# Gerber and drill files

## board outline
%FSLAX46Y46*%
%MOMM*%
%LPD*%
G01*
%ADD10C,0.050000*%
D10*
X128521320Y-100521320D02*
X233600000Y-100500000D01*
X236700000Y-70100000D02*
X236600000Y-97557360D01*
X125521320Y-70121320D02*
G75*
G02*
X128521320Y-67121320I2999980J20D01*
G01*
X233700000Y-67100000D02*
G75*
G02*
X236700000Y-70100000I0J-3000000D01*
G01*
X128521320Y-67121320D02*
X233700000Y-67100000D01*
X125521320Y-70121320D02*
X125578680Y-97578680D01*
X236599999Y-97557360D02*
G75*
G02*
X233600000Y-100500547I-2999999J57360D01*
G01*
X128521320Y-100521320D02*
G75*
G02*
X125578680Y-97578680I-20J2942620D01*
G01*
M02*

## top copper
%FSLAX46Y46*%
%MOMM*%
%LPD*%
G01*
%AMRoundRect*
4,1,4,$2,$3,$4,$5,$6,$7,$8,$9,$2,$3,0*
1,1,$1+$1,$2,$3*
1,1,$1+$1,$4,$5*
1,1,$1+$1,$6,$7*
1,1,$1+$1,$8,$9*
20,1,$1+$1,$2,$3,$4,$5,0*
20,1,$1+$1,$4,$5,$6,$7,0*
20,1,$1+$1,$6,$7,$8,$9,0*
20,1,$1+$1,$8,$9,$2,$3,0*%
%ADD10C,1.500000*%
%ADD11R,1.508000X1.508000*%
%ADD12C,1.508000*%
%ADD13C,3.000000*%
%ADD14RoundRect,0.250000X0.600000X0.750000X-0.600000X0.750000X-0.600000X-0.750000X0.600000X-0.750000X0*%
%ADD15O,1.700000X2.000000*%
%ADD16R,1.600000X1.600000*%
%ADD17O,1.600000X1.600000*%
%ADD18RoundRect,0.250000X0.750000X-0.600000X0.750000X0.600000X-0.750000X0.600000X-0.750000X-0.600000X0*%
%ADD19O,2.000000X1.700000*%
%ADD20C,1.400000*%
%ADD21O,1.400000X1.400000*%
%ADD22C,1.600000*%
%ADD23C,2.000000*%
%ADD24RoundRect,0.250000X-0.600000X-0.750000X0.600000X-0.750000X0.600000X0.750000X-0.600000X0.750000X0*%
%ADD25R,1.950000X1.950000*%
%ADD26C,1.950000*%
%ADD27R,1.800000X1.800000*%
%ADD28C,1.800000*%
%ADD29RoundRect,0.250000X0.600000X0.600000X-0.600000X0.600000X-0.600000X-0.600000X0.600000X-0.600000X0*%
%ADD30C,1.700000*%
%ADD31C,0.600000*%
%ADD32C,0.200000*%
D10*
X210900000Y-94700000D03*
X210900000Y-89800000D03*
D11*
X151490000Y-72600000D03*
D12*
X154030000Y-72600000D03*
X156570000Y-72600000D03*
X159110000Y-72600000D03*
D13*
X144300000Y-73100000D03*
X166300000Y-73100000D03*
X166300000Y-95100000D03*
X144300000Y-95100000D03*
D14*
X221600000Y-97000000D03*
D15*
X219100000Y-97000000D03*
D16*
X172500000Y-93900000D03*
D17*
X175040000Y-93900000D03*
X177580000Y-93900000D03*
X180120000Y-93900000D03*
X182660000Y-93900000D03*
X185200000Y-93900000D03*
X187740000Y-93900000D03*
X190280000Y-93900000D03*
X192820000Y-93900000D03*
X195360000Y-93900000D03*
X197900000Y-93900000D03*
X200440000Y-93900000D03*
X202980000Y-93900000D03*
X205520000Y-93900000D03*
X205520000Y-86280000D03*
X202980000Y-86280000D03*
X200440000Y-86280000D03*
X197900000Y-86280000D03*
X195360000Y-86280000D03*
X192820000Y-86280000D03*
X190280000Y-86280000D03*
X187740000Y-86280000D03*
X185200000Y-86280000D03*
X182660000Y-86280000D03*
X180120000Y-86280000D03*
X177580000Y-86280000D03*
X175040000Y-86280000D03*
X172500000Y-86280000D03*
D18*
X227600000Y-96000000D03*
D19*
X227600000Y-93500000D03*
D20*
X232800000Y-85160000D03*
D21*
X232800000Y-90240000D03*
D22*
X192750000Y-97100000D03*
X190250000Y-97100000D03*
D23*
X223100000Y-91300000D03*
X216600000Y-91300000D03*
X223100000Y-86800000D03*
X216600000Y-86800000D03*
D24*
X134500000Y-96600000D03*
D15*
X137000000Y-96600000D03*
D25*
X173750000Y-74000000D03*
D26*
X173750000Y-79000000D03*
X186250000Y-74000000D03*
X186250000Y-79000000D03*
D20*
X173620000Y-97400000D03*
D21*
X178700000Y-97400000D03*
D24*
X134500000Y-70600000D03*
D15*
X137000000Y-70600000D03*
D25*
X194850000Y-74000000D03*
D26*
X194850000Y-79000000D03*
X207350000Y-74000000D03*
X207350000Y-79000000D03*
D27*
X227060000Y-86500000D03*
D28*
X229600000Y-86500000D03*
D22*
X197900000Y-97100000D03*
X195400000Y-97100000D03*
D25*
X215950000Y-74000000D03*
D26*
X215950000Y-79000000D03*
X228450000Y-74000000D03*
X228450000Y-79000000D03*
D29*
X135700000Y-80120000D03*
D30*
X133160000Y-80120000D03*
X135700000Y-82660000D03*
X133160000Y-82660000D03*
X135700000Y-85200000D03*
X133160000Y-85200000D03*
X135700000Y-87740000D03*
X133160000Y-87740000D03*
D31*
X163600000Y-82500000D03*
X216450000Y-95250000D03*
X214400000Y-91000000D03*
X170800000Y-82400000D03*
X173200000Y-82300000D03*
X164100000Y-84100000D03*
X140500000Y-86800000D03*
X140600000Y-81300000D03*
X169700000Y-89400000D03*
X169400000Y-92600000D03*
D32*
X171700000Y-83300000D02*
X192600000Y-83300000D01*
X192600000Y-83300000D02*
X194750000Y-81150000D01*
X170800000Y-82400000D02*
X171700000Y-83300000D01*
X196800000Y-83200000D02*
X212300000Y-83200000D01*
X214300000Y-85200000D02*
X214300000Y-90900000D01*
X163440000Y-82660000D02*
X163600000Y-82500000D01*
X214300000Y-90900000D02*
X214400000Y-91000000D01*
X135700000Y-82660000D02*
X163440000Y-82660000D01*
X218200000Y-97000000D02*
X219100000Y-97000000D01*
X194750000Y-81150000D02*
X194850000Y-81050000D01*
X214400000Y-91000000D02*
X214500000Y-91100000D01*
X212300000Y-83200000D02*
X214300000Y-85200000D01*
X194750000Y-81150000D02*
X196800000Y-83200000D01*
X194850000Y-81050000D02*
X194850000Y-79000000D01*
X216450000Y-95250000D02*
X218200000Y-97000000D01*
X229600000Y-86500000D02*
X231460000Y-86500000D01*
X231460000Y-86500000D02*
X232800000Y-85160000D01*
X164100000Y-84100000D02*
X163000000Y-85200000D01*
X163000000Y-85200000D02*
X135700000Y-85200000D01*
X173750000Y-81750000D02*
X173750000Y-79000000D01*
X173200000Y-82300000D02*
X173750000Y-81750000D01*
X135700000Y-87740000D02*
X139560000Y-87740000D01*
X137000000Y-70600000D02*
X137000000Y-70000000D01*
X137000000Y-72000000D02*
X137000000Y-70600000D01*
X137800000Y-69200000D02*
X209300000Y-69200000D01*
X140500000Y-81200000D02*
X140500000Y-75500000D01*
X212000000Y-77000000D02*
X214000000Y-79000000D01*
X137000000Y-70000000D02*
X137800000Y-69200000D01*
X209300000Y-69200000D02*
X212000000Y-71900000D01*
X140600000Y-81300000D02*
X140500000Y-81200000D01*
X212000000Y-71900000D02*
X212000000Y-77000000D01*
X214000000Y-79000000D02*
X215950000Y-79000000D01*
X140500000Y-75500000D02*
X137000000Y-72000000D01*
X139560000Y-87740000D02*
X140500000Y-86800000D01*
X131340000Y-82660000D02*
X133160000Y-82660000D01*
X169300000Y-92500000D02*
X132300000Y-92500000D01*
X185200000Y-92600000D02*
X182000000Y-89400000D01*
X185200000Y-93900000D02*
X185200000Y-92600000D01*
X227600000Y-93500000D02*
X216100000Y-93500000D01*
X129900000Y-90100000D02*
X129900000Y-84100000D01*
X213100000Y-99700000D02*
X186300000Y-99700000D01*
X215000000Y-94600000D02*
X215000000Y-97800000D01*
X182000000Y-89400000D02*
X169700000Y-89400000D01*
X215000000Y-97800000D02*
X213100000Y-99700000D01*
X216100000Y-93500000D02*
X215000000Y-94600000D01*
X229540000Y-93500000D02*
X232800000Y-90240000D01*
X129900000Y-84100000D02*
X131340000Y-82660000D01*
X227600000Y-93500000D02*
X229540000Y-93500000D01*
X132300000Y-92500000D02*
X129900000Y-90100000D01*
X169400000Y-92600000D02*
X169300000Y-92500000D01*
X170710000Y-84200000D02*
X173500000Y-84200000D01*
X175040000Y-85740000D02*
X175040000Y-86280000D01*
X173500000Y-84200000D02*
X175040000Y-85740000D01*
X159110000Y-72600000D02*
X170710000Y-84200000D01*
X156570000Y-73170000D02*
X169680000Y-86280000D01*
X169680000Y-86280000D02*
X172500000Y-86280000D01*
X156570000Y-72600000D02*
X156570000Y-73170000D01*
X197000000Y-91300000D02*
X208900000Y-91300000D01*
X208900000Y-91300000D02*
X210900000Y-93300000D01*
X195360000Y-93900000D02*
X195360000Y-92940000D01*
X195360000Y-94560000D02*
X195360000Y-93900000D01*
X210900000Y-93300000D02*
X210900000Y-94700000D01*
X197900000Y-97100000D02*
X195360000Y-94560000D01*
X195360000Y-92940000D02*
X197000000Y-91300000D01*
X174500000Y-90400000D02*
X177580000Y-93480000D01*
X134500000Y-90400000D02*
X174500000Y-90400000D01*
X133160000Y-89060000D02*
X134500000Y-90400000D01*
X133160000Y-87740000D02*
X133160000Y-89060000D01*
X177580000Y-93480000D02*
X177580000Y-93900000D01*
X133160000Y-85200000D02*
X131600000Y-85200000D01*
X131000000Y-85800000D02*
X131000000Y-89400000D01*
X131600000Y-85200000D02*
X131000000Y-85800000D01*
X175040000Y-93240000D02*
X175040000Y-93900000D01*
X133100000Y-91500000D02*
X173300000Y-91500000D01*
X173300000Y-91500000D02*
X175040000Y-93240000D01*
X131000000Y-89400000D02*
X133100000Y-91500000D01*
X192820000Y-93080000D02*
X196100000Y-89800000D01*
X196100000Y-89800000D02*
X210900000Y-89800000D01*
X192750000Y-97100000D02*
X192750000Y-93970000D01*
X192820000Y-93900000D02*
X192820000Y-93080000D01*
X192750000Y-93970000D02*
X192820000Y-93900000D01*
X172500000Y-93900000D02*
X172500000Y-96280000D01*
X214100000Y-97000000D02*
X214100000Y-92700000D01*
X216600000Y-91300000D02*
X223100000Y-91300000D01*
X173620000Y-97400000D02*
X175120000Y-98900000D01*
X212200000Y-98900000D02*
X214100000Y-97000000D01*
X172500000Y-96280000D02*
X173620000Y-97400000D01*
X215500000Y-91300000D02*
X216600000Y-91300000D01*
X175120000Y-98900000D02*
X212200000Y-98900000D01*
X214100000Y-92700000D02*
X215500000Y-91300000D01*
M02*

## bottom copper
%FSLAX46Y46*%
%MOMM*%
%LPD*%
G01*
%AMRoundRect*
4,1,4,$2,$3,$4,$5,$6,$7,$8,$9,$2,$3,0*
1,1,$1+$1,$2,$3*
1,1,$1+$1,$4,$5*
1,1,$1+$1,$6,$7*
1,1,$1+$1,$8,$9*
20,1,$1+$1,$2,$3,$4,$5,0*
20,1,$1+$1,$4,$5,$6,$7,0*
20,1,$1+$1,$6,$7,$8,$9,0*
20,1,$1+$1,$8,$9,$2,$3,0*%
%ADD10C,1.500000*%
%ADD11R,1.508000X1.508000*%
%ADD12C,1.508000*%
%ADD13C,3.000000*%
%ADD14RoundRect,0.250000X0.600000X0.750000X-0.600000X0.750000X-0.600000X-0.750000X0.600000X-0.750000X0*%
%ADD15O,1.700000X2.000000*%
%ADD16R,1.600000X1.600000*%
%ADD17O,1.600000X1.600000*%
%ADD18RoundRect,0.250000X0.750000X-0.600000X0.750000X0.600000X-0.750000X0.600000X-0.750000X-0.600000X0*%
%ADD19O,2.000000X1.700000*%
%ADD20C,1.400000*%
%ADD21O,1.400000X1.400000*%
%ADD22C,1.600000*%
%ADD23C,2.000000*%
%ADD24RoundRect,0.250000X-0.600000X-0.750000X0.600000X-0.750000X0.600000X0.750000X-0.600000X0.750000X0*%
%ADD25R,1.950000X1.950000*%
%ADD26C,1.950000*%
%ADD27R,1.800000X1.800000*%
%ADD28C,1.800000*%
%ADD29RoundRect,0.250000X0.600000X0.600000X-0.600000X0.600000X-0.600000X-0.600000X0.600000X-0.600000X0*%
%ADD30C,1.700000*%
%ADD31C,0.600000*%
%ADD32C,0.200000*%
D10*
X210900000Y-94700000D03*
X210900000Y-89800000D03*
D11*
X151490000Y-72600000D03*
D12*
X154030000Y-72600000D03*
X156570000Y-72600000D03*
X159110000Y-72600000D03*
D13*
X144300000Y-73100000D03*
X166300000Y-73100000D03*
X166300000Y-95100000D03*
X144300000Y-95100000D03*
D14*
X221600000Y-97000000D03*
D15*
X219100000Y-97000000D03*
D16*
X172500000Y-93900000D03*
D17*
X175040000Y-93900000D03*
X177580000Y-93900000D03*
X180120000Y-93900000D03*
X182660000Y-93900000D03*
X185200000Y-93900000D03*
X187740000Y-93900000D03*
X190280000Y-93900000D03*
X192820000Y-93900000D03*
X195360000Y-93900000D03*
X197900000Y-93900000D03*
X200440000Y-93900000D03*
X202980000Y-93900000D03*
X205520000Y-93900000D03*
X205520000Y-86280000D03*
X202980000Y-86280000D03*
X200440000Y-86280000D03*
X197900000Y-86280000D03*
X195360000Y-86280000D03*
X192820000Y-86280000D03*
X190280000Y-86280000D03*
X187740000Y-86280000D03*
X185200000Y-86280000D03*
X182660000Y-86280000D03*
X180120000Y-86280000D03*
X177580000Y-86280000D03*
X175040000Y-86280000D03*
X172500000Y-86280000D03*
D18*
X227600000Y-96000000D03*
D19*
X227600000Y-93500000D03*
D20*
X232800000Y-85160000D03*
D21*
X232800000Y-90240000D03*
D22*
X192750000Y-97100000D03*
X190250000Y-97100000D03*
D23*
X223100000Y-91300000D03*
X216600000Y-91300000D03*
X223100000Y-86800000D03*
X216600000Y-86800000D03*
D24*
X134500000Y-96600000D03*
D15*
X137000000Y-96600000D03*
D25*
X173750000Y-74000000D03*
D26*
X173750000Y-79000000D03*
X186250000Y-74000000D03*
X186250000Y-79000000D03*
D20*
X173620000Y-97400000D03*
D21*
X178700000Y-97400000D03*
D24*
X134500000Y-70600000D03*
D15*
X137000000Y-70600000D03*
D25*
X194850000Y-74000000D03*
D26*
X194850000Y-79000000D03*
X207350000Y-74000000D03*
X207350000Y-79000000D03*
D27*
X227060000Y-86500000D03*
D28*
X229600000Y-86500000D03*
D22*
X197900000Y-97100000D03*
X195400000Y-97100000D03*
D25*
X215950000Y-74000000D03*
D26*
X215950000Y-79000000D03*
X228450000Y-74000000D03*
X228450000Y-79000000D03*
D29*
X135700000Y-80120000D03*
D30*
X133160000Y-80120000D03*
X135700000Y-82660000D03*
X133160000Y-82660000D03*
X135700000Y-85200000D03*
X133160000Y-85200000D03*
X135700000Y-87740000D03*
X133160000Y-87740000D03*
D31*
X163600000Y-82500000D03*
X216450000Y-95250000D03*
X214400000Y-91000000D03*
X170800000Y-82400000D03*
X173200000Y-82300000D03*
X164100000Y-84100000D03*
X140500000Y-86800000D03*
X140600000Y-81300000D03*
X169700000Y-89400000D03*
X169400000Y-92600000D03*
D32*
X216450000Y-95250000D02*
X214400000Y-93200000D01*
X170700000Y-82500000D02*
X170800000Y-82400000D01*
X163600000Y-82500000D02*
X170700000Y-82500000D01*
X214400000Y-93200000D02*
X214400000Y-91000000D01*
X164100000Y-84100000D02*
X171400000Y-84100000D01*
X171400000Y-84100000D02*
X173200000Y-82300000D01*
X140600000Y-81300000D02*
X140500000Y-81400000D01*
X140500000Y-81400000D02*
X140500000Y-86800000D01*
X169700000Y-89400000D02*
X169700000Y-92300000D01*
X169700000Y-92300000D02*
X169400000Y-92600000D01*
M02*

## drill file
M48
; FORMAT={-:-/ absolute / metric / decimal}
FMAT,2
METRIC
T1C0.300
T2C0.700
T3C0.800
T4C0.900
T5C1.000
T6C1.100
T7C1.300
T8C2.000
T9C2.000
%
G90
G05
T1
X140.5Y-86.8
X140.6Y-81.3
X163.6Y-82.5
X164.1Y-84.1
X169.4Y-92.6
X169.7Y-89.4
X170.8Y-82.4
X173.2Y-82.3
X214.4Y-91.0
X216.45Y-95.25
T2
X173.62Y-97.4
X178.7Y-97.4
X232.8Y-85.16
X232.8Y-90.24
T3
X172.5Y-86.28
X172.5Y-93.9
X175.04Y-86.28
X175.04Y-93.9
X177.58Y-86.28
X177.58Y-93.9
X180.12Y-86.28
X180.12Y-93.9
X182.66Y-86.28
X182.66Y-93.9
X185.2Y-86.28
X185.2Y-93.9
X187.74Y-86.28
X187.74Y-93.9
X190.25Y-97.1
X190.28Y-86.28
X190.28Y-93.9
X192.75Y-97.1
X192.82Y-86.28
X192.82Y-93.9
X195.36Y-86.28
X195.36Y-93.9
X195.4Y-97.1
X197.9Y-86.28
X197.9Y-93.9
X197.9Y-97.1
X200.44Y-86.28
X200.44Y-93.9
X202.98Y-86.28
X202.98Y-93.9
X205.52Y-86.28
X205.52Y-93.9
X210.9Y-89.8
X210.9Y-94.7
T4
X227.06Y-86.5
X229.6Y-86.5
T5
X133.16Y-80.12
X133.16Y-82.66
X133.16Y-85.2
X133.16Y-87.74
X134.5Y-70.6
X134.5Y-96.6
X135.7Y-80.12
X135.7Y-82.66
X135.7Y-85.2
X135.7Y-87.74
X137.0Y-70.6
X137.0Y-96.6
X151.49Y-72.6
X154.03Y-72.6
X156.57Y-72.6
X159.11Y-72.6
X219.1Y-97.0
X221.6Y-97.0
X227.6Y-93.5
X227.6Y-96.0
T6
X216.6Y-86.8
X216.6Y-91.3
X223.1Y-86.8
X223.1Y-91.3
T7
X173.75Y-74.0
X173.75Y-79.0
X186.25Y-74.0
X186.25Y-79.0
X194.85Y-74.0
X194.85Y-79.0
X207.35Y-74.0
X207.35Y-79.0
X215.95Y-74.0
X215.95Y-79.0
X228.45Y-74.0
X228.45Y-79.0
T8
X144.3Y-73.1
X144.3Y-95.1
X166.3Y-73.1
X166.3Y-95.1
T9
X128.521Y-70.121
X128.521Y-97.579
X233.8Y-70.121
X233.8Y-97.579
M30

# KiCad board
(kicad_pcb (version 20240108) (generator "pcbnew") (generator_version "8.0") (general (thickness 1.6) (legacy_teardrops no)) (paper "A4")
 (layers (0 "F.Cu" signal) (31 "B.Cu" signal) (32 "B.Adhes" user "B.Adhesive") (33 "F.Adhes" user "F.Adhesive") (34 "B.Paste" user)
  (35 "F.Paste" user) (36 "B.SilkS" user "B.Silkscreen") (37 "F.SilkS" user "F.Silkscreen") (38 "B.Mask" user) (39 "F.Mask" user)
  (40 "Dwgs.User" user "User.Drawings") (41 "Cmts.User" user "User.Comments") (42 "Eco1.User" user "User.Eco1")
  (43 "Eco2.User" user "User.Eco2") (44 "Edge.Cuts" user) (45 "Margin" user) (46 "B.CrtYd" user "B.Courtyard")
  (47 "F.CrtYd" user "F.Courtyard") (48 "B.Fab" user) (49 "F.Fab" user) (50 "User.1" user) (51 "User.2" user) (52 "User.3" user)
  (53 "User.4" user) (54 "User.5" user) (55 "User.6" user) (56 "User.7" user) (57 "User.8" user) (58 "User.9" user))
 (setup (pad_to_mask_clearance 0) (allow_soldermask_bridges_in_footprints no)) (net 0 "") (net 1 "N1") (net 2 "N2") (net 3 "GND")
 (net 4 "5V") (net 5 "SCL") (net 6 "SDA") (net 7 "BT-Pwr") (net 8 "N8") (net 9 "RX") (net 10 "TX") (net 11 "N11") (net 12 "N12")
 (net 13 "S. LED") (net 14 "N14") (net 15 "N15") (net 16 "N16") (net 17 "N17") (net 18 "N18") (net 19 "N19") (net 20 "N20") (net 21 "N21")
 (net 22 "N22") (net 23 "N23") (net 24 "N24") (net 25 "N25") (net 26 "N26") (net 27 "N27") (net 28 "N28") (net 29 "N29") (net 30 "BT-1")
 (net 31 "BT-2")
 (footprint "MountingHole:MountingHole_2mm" (layer "F.Cu") (at 233.8 97.5787)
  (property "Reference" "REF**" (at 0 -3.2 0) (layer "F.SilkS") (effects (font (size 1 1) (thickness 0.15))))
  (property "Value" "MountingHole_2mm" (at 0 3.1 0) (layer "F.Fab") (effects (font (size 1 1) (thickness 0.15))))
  (pad "" np_thru_hole circle (at 0 0) (size 2 2) (drill 2) (layers "*.Cu" "*.Mask")))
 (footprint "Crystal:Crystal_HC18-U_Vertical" (layer "F.Cu") (at 210.9 94.7 90)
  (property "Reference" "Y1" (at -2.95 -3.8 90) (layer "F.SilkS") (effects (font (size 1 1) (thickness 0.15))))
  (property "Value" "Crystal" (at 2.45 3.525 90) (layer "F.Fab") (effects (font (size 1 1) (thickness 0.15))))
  (pad "1" thru_hole circle (at 0 0 90) (size 1.5 1.5) (drill 0.8) (layers "*.Cu" "*.Mask") (remove_unused_layers no) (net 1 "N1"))
  (pad "2" thru_hole circle (at 4.9 0 90) (size 1.5 1.5) (drill 0.8) (layers "*.Cu" "*.Mask") (remove_unused_layers no) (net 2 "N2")))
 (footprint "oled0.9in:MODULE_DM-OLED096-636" (layer "F.Cu") (at 155.3 84.1)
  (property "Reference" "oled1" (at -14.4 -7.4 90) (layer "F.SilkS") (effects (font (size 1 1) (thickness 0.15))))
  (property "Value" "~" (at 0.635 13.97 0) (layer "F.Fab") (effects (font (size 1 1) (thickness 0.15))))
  (pad "1" thru_hole rect (at -3.81 -11.5) (size 1.508 1.508) (drill 1) (layers "*.Cu" "*.Mask") (remove_unused_layers no) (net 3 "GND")
   (solder_mask_margin 0.102))
  (pad "2" thru_hole circle (at -1.27 -11.5) (size 1.508 1.508) (drill 1) (layers "*.Cu" "*.Mask") (remove_unused_layers no) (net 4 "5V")
   (solder_mask_margin 0.102))
  (pad "3" thru_hole circle (at 1.27 -11.5) (size 1.508 1.508) (drill 1) (layers "*.Cu" "*.Mask") (remove_unused_layers no) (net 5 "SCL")
   (solder_mask_margin 0.102))
  (pad "4" thru_hole circle (at 3.81 -11.5) (size 1.508 1.508) (drill 1) (layers "*.Cu" "*.Mask") (remove_unused_layers no) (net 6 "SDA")
   (solder_mask_margin 0.102))
  (pad "S1" thru_hole circle (at -11 -11) (size 3 3) (drill 2) (layers "*.Cu" "*.Mask") (remove_unused_layers no) (solder_mask_margin 0.102))
  (pad "S2" thru_hole circle (at 11 -11) (size 3 3) (drill 2) (layers "*.Cu" "*.Mask") (remove_unused_layers no) (solder_mask_margin 0.102))
  (pad "S3" thru_hole circle (at 11 11) (size 3 3) (drill 2) (layers "*.Cu" "*.Mask") (remove_unused_layers no) (solder_mask_margin 0.102))
  (pad "S4" thru_hole circle (at -11 11) (size 3 3) (drill 2) (layers "*.Cu" "*.Mask") (remove_unused_layers no) (solder_mask_margin 0.102)))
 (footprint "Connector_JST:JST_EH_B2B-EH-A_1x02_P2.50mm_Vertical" (layer "F.Cu") (at 221.6 97 180)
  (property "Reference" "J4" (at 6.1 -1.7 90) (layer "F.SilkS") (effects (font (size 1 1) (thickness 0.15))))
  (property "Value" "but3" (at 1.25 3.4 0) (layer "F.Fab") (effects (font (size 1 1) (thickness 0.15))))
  (pad "1" thru_hole roundrect (at 0 0 180) (size 1.7 2) (drill 1) (layers "*.Cu" "*.Mask") (remove_unused_layers no)
   (roundrect_rratio 0.147059) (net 3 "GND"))
  (pad "2" thru_hole oval (at 2.5 0 180) (size 1.7 2) (drill 1) (layers "*.Cu" "*.Mask") (remove_unused_layers no) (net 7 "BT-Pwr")))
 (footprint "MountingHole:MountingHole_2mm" (layer "F.Cu") (at 128.5213 97.5787)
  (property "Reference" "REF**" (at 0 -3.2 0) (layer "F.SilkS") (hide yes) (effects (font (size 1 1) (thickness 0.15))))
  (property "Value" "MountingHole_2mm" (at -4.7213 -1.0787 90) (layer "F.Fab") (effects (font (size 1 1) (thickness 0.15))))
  (pad "" np_thru_hole circle (at 0 0) (size 2 2) (drill 2) (layers "*.Cu" "*.Mask")))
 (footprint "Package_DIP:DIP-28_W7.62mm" (layer "F.Cu") (at 172.5 93.9 90)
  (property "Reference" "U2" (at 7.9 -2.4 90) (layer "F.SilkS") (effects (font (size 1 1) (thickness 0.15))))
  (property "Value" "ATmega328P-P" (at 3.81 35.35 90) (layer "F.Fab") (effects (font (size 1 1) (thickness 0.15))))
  (pad "1" thru_hole rect (at 0 0 90) (size 1.6 1.6) (drill 0.8) (layers "*.Cu" "*.Mask") (remove_unused_layers no) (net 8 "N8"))
  (pad "2" thru_hole oval (at 0 2.54 90) (size 1.6 1.6) (drill 0.8) (layers "*.Cu" "*.Mask") (remove_unused_layers no) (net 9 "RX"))
  (pad "3" thru_hole oval (at 0 5.08 90) (size 1.6 1.6) (drill 0.8) (layers "*.Cu" "*.Mask") (remove_unused_layers no) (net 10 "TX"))
  (pad "4" thru_hole oval (at 0 7.62 90) (size 1.6 1.6) (drill 0.8) (layers "*.Cu" "*.Mask") (remove_unused_layers no) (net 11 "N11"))
  (pad "5" thru_hole oval (at 0 10.16 90) (size 1.6 1.6) (drill 0.8) (layers "*.Cu" "*.Mask") (remove_unused_layers no) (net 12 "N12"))
  (pad "6" thru_hole oval (at 0 12.7 90) (size 1.6 1.6) (drill 0.8) (layers "*.Cu" "*.Mask") (remove_unused_layers no) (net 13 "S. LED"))
  (pad "7" thru_hole oval (at 0 15.24 90) (size 1.6 1.6) (drill 0.8) (layers "*.Cu" "*.Mask") (remove_unused_layers no) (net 4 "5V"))
  (pad "8" thru_hole oval (at 0 17.78 90) (size 1.6 1.6) (drill 0.8) (layers "*.Cu" "*.Mask") (remove_unused_layers no) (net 3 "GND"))
  (pad "9" thru_hole oval (at 0 20.32 90) (size 1.6 1.6) (drill 0.8) (layers "*.Cu" "*.Mask") (remove_unused_layers no) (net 2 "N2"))
  (pad "10" thru_hole oval (at 0 22.86 90) (size 1.6 1.6) (drill 0.8) (layers "*.Cu" "*.Mask") (remove_unused_layers no) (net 1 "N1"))
  (pad "11" thru_hole oval (at 0 25.4 90) (size 1.6 1.6) (drill 0.8) (layers "*.Cu" "*.Mask") (remove_unused_layers no) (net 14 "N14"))
  (pad "12" thru_hole oval (at 0 27.94 90) (size 1.6 1.6) (drill 0.8) (layers "*.Cu" "*.Mask") (remove_unused_layers no) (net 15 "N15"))
  (pad "13" thru_hole oval (at 0 30.48 90) (size 1.6 1.6) (drill 0.8) (layers "*.Cu" "*.Mask") (remove_unused_layers no) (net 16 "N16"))
  (pad "14" thru_hole oval (at 0 33.02 90) (size 1.6 1.6) (drill 0.8) (layers "*.Cu" "*.Mask") (remove_unused_layers no) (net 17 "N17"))
  (pad "15" thru_hole oval (at 7.62 33.02 90) (size 1.6 1.6) (drill 0.8) (layers "*.Cu" "*.Mask") (remove_unused_layers no) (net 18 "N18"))
  (pad "16" thru_hole oval (at 7.62 30.48 90) (size 1.6 1.6) (drill 0.8) (layers "*.Cu" "*.Mask") (remove_unused_layers no) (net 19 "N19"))
  (pad "17" thru_hole oval (at 7.62 27.94 90) (size 1.6 1.6) (drill 0.8) (layers "*.Cu" "*.Mask") (remove_unused_layers no) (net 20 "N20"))
  (pad "18" thru_hole oval (at 7.62 25.4 90) (size 1.6 1.6) (drill 0.8) (layers "*.Cu" "*.Mask") (remove_unused_layers no) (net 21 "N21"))
  (pad "19" thru_hole oval (at 7.62 22.86 90) (size 1.6 1.6) (drill 0.8) (layers "*.Cu" "*.Mask") (remove_unused_layers no) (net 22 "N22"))
  (pad "20" thru_hole oval (at 7.62 20.32 90) (size 1.6 1.6) (drill 0.8) (layers "*.Cu" "*.Mask") (remove_unused_layers no) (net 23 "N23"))
  (pad "21" thru_hole oval (at 7.62 17.78 90) (size 1.6 1.6) (drill 0.8) (layers "*.Cu" "*.Mask") (remove_unused_layers no) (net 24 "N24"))
  (pad "22" thru_hole oval (at 7.62 15.24 90) (size 1.6 1.6) (drill 0.8) (layers "*.Cu" "*.Mask") (remove_unused_layers no) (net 3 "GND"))
  (pad "23" thru_hole oval (at 7.62 12.7 90) (size 1.6 1.6) (drill 0.8) (layers "*.Cu" "*.Mask") (remove_unused_layers no) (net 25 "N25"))
  (pad "24" thru_hole oval (at 7.62 10.16 90) (size 1.6 1.6) (drill 0.8) (layers "*.Cu" "*.Mask") (remove_unused_layers no) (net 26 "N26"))
  (pad "25" thru_hole oval (at 7.62 7.62 90) (size 1.6 1.6) (drill 0.8) (layers "*.Cu" "*.Mask") (remove_unused_layers no) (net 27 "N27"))
  (pad "26" thru_hole oval (at 7.62 5.08 90) (size 1.6 1.6) (drill 0.8) (layers "*.Cu" "*.Mask") (remove_unused_layers no) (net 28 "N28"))
  (pad "27" thru_hole oval (at 7.62 2.54 90) (size 1.6 1.6) (drill 0.8) (layers "*.Cu" "*.Mask") (remove_unused_layers no) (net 6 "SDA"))
  (pad "28" thru_hole oval (at 7.62 0 90) (size 1.6 1.6) (drill 0.8) (layers "*.Cu" "*.Mask") (remove_unused_layers no) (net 5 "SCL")))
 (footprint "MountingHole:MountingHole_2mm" (layer "F.Cu") (at 233.8 70.1213)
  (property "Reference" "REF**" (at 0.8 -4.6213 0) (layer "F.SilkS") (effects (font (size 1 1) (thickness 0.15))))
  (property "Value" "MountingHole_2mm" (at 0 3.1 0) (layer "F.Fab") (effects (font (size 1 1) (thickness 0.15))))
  (pad "" np_thru_hole circle (at 0 0) (size 2 2) (drill 2) (layers "*.Cu" "*.Mask")))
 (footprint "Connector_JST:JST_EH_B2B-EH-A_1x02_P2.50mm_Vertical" (layer "F.Cu") (at 227.6 96 90)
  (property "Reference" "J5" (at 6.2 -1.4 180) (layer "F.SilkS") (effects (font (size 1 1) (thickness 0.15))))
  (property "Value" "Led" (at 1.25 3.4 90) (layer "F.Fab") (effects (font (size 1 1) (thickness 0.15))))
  (pad "1" thru_hole roundrect (at 0 0 90) (size 1.7 2) (drill 1) (layers "*.Cu" "*.Mask") (remove_unused_layers no)
   (roundrect_rratio 0.147059) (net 3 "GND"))
  (pad "2" thru_hole oval (at 2.5 0 90) (size 1.7 2) (drill 1) (layers "*.Cu" "*.Mask") (remove_unused_layers no) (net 13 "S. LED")))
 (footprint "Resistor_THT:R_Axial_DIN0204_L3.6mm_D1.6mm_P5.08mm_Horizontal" (layer "F.Cu") (at 232.8 85.16 -90)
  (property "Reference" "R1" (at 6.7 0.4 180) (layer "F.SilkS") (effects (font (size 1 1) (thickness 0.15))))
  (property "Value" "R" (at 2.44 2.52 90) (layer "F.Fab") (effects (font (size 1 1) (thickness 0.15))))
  (pad "1" thru_hole circle (at 0 0 270) (size 1.4 1.4) (drill 0.7) (layers "*.Cu" "*.Mask") (remove_unused_layers no) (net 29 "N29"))
  (pad "2" thru_hole oval (at 5.08 0 270) (size 1.4 1.4) (drill 0.7) (layers "*.Cu" "*.Mask") (remove_unused_layers no) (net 13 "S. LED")))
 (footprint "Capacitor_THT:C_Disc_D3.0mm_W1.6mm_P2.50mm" (layer "F.Cu") (at 192.75 97.1 180)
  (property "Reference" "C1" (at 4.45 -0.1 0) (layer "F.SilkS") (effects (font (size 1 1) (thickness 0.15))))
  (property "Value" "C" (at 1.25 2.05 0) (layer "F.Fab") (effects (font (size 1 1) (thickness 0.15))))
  (pad "1" thru_hole circle (at 0 0 180) (size 1.6 1.6) (drill 0.8) (layers "*.Cu" "*.Mask") (remove_unused_layers no) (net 2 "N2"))
  (pad "2" thru_hole circle (at 2.5 0 180) (size 1.6 1.6) (drill 0.8) (layers "*.Cu" "*.Mask") (remove_unused_layers no) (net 3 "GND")))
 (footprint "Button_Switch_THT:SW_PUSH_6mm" (layer "F.Cu") (at 223.1 91.3 180)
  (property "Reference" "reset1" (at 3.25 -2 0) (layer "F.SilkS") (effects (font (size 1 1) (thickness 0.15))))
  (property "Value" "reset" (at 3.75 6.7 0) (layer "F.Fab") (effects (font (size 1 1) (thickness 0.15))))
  (pad "1" thru_hole circle (at 0 0 270) (size 2 2) (drill 1.1) (layers "*.Cu" "*.Mask") (remove_unused_layers no) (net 8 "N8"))
  (pad "1" thru_hole circle (at 6.5 0 270) (size 2 2) (drill 1.1) (layers "*.Cu" "*.Mask") (remove_unused_layers no) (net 8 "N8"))
  (pad "2" thru_hole circle (at 0 4.5 270) (size 2 2) (drill 1.1) (layers "*.Cu" "*.Mask") (remove_unused_layers no) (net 3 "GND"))
  (pad "2" thru_hole circle (at 6.5 4.5 270) (size 2 2) (drill 1.1) (layers "*.Cu" "*.Mask") (remove_unused_layers no) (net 3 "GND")))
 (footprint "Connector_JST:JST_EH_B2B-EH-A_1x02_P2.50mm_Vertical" (layer "F.Cu") (at 134.5 96.6)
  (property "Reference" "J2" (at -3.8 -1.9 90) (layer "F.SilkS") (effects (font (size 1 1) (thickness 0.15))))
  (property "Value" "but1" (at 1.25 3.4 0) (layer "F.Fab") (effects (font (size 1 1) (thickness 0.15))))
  (pad "1" thru_hole roundrect (at 0 0) (size 1.7 2) (drill 1) (layers "*.Cu" "*.Mask") (remove_unused_layers no)
   (roundrect_rratio 0.147059) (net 3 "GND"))
  (pad "2" thru_hole oval (at 2.5 0) (size 1.7 2) (drill 1) (layers "*.Cu" "*.Mask") (remove_unused_layers no) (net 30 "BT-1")))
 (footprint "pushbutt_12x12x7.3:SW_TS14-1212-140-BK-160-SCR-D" (layer "F.Cu") (at 180 76.5)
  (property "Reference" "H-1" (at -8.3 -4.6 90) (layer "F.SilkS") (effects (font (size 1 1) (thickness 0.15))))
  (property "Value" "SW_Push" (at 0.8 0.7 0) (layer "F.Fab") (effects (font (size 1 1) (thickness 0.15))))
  (pad "1" thru_hole rect (at -6.25 -2.5) (size 1.95 1.95) (drill 1.3) (layers "*.Cu" "*.Mask") (remove_unused_layers no) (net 3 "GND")
   (solder_mask_margin 0.102))
  (pad "2" thru_hole circle (at -6.25 2.5) (size 1.95 1.95) (drill 1.3) (layers "*.Cu" "*.Mask") (remove_unused_layers no) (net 30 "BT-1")
   (solder_mask_margin 0.102))
  (pad "3" thru_hole circle (at 6.25 -2.5) (size 1.95 1.95) (drill 1.3) (layers "*.Cu" "*.Mask") (remove_unused_layers no)
   (solder_mask_margin 0.102))
  (pad "4" thru_hole circle (at 6.25 2.5) (size 1.95 1.95) (drill 1.3) (layers "*.Cu" "*.Mask") (remove_unused_layers no)
   (solder_mask_margin 0.102)))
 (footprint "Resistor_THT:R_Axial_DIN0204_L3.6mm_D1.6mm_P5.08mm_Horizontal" (layer "F.Cu") (at 173.62 97.4)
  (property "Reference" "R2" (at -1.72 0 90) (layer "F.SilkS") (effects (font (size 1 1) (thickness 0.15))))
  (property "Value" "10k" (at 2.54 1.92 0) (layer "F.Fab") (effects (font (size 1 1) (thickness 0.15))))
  (pad "1" thru_hole circle (at 0 0) (size 1.4 1.4) (drill 0.7) (layers "*.Cu" "*.Mask") (remove_unused_layers no) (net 8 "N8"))
  (pad "2" thru_hole oval (at 5.08 0) (size 1.4 1.4) (drill 0.7) (layers "*.Cu" "*.Mask") (remove_unused_layers no) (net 4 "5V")))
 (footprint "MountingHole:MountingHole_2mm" (layer "F.Cu") (at 128.5213 70.1213)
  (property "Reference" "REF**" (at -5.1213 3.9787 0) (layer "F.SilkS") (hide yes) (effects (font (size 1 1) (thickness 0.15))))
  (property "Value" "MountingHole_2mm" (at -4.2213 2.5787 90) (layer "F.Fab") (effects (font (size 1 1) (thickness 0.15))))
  (pad "" np_thru_hole circle (at 0 0) (size 2 2) (drill 2) (layers "*.Cu" "*.Mask")))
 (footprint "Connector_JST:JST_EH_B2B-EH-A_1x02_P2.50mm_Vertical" (layer "F.Cu") (at 134.5 70.6)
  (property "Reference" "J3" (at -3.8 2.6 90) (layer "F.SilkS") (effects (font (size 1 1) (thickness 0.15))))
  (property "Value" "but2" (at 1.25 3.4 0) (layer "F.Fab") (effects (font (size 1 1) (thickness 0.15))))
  (pad "1" thru_hole roundrect (at 0 0) (size 1.7 2) (drill 1) (layers "*.Cu" "*.Mask") (remove_unused_layers no)
   (roundrect_rratio 0.147059) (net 3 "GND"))
  (pad "2" thru_hole oval (at 2.5 0) (size 1.7 2) (drill 1) (layers "*.Cu" "*.Mask") (remove_unused_layers no) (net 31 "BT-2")))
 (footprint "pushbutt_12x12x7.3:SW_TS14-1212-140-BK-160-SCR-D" (layer "F.Cu") (at 201.1 76.5)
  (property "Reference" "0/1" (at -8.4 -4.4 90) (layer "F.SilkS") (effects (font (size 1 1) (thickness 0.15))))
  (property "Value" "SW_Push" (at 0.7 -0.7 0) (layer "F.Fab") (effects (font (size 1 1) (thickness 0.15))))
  (pad "1" thru_hole rect (at -6.25 -2.5) (size 1.95 1.95) (drill 1.3) (layers "*.Cu" "*.Mask") (remove_unused_layers no) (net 3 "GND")
   (solder_mask_margin 0.102))
  (pad "2" thru_hole circle (at -6.25 2.5) (size 1.95 1.95) (drill 1.3) (layers "*.Cu" "*.Mask") (remove_unused_layers no) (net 7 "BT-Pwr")
   (solder_mask_margin 0.102))
  (pad "3" thru_hole circle (at 6.25 -2.5) (size 1.95 1.95) (drill 1.3) (layers "*.Cu" "*.Mask") (remove_unused_layers no)
   (solder_mask_margin 0.102))
  (pad "4" thru_hole circle (at 6.25 2.5) (size 1.95 1.95) (drill 1.3) (layers "*.Cu" "*.Mask") (remove_unused_layers no)
   (solder_mask_margin 0.102)))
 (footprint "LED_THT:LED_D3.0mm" (layer "F.Cu") (at 227.06 86.5)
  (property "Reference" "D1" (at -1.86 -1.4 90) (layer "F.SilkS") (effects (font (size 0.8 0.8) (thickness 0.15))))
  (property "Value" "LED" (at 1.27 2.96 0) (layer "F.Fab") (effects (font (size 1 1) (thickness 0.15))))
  (pad "1" thru_hole rect (at 0 0) (size 1.8 1.8) (drill 0.9) (layers "*.Cu" "*.Mask") (remove_unused_layers no) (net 3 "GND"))
  (pad "2" thru_hole circle (at 2.54 0) (size 1.8 1.8) (drill 0.9) (layers "*.Cu" "*.Mask") (remove_unused_layers no) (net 29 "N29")))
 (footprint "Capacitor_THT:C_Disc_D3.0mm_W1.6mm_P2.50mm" (layer "F.Cu") (at 197.9 97.1 180)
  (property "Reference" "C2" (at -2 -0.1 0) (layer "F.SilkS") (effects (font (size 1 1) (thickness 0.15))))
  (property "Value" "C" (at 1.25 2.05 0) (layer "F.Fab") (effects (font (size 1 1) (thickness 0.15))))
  (pad "1" thru_hole circle (at 0 0 180) (size 1.6 1.6) (drill 0.8) (layers "*.Cu" "*.Mask") (remove_unused_layers no) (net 1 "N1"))
  (pad "2" thru_hole circle (at 2.5 0 180) (size 1.6 1.6) (drill 0.8) (layers "*.Cu" "*.Mask") (remove_unused_layers no) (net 3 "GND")))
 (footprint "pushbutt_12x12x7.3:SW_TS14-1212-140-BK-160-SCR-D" (layer "F.Cu") (at 222.2 76.5)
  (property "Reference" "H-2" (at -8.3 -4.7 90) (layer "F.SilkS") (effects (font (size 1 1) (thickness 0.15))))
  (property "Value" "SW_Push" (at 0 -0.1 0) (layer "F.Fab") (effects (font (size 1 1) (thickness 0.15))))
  (pad "1" thru_hole rect (at -6.25 -2.5) (size 1.95 1.95) (drill 1.3) (layers "*.Cu" "*.Mask") (remove_unused_layers no) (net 3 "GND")
   (solder_mask_margin 0.102))
  (pad "2" thru_hole circle (at -6.25 2.5) (size 1.95 1.95) (drill 1.3) (layers "*.Cu" "*.Mask") (remove_unused_layers no) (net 31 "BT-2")
   (solder_mask_margin 0.102))
  (pad "3" thru_hole circle (at 6.25 -2.5) (size 1.95 1.95) (drill 1.3) (layers "*.Cu" "*.Mask") (remove_unused_layers no)
   (solder_mask_margin 0.102))
  (pad "4" thru_hole circle (at 6.25 2.5) (size 1.95 1.95) (drill 1.3) (layers "*.Cu" "*.Mask") (remove_unused_layers no)
   (solder_mask_margin 0.102)))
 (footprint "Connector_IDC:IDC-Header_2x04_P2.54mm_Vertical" (layer "B.Cu") (at 135.7 80.12 180)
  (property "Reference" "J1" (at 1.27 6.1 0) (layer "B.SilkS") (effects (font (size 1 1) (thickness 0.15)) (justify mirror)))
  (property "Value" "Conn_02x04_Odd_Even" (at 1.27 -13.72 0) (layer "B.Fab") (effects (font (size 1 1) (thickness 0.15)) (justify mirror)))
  (pad "1" thru_hole roundrect (at 0 0 180) (size 1.7 1.7) (drill 1) (layers "*.Cu" "*.Mask") (remove_unused_layers no)
   (roundrect_rratio 0.147059) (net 4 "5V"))
  (pad "2" thru_hole circle (at 2.54 0 180) (size 1.7 1.7) (drill 1) (layers "*.Cu" "*.Mask") (remove_unused_layers no) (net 3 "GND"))
  (pad "3" thru_hole circle (at 0 -2.54 180) (size 1.7 1.7) (drill 1) (layers "*.Cu" "*.Mask") (remove_unused_layers no) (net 7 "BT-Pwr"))
  (pad "4" thru_hole circle (at 2.54 -2.54 180) (size 1.7 1.7) (drill 1) (layers "*.Cu" "*.Mask") (remove_unused_layers no)
   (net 13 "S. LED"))
  (pad "5" thru_hole circle (at 0 -5.08 180) (size 1.7 1.7) (drill 1) (layers "*.Cu" "*.Mask") (remove_unused_layers no) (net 30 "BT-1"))
  (pad "6" thru_hole circle (at 2.54 -5.08 180) (size 1.7 1.7) (drill 1) (layers "*.Cu" "*.Mask") (remove_unused_layers no) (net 9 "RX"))
  (pad "7" thru_hole circle (at 0 -7.62 180) (size 1.7 1.7) (drill 1) (layers "*.Cu" "*.Mask") (remove_unused_layers no) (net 31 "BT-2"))
  (pad "8" thru_hole circle (at 2.54 -7.62 180) (size 1.7 1.7) (drill 1) (layers "*.Cu" "*.Mask") (remove_unused_layers no) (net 10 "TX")))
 (gr_line (start 128.52132 100.52132) (end 233.6 100.5) (stroke (width 0.05) (type default)) (layer "Edge.Cuts"))
 (gr_line (start 236.7 70.1) (end 236.6 97.55736) (stroke (width 0.05) (type default)) (layer "Edge.Cuts"))
 (gr_arc (start 125.52132 70.12132) (mid 126.4 68) (end 128.52132 67.12132) (stroke (width 0.05) (type default)) (layer "Edge.Cuts"))
 (gr_arc (start 233.7 67.1) (mid 235.821326 67.978674) (end 236.7 70.1) (stroke (width 0.05) (type default)) (layer "Edge.Cuts"))
 (gr_line (start 128.52132 67.12132) (end 233.7 67.1) (stroke (width 0.05) (type default)) (layer "Edge.Cuts"))
 (gr_line (start 125.52132 70.12132) (end 125.57868 97.57868) (stroke (width 0.05) (type default)) (layer "Edge.Cuts"))
 (gr_arc (start 236.599999 97.55736) (mid 235.701343 99.641917) (end 233.6 100.500587) (stroke (width 0.05) (type default))
  (layer "Edge.Cuts"))
 (gr_arc (start 128.52132 100.52132) (mid 126.440553 99.659447) (end 125.57868 97.57868) (stroke (width 0.05) (type default))
  (layer "Edge.Cuts"))
 (segment (start 171.7 83.3) (end 192.6 83.3) (width 0.2) (layer "F.Cu") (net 7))
 (segment (start 192.6 83.3) (end 194.75 81.15) (width 0.2) (layer "F.Cu") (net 7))
 (segment (start 170.8 82.4) (end 171.7 83.3) (width 0.2) (layer "F.Cu") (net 7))
 (segment (start 196.8 83.2) (end 212.3 83.2) (width 0.2) (layer "F.Cu") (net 7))
 (segment (start 214.3 85.2) (end 214.3 90.9) (width 0.2) (layer "F.Cu") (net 7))
 (segment (start 163.44 82.66) (end 163.6 82.5) (width 0.2) (layer "F.Cu") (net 7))
 (segment (start 214.3 90.9) (end 214.4 91) (width 0.2) (layer "F.Cu") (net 7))
 (segment (start 135.7 82.66) (end 163.44 82.66) (width 0.2) (layer "F.Cu") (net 7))
 (segment (start 218.2 97) (end 219.1 97) (width 0.2) (layer "F.Cu") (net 7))
 (segment (start 194.75 81.15) (end 194.85 81.05) (width 0.2) (layer "F.Cu") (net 7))
 (segment (start 214.4 91) (end 214.5 91.1) (width 0.2) (layer "F.Cu") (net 7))
 (segment (start 212.3 83.2) (end 214.3 85.2) (width 0.2) (layer "F.Cu") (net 7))
 (segment (start 194.75 81.15) (end 196.8 83.2) (width 0.2) (layer "F.Cu") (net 7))
 (segment (start 194.85 81.05) (end 194.85 79) (width 0.2) (layer "F.Cu") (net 7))
 (segment (start 216.45 95.25) (end 218.2 97) (width 0.2) (layer "F.Cu") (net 7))
 (via (at 163.6 82.5) (size 0.6) (drill 0.3) (layers "F.Cu" "B.Cu") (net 7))
 (via (at 216.45 95.25) (size 0.6) (drill 0.3) (layers "F.Cu" "B.Cu") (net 7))
 (via (at 214.4 91) (size 0.6) (drill 0.3) (layers "F.Cu" "B.Cu") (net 7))
 (via (at 170.8 82.4) (size 0.6) (drill 0.3) (layers "F.Cu" "B.Cu") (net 7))
 (segment (start 216.45 95.25) (end 214.4 93.2) (width 0.2) (layer "B.Cu") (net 7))
 (segment (start 170.7 82.5) (end 170.8 82.4) (width 0.2) (layer "B.Cu") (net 7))
 (segment (start 163.6 82.5) (end 170.7 82.5) (width 0.2) (layer "B.Cu") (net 7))
 (segment (start 214.4 93.2) (end 214.4 91) (width 0.2) (layer "B.Cu") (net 7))
 (segment (start 229.6 86.5) (end 231.46 86.5) (width 0.2) (layer "F.Cu") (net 29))
 (segment (start 231.46 86.5) (end 232.8 85.16) (width 0.2) (layer "F.Cu") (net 29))
 (segment (start 164.1 84.1) (end 163 85.2) (width 0.2) (layer "F.Cu") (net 30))
 (segment (start 163 85.2) (end 135.7 85.2) (width 0.2) (layer "F.Cu") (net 30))
 (segment (start 173.75 81.75) (end 173.75 79) (width 0.2) (layer "F.Cu") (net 30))
 (segment (start 173.2 82.3) (end 173.75 81.75) (width 0.2) (layer "F.Cu") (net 30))
 (via (at 173.2 82.3) (size 0.6) (drill 0.3) (layers "F.Cu" "B.Cu") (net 30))
 (via (at 164.1 84.1) (size 0.6) (drill 0.3) (layers "F.Cu" "B.Cu") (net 30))
 (segment (start 164.1 84.1) (end 171.4 84.1) (width 0.2) (layer "B.Cu") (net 30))
 (segment (start 171.4 84.1) (end 173.2 82.3) (width 0.2) (layer "B.Cu") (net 30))
 (segment (start 135.7 87.74) (end 139.56 87.74) (width 0.2) (layer "F.Cu") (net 31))
 (segment (start 137 70.6) (end 137 70) (width 0.2) (layer "F.Cu") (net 31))
 (segment (start 137 72) (end 137 70.6) (width 0.2) (layer "F.Cu") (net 31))
 (segment (start 137.8 69.2) (end 209.3 69.2) (width 0.2) (layer "F.Cu") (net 31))
 (segment (start 140.5 81.2) (end 140.5 75.5) (width 0.2) (layer "F.Cu") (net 31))
 (segment (start 212 77) (end 214 79) (width 0.2) (layer "F.Cu") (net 31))
 (segment (start 137 70) (end 137.8 69.2) (width 0.2) (layer "F.Cu") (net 31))
 (segment (start 209.3 69.2) (end 212 71.9) (width 0.2) (layer "F.Cu") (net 31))
 (segment (start 140.6 81.3) (end 140.5 81.2) (width 0.2) (layer "F.Cu") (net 31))
 (segment (start 212 71.9) (end 212 77) (width 0.2) (layer "F.Cu") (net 31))
 (segment (start 214 79) (end 215.95 79) (width 0.2) (layer "F.Cu") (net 31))
 (segment (start 140.5 75.5) (end 137 72) (width 0.2) (layer "F.Cu") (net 31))
 (segment (start 139.56 87.74) (end 140.5 86.8) (width 0.2) (layer "F.Cu") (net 31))
 (via (at 140.5 86.8) (size 0.6) (drill 0.3) (layers "F.Cu" "B.Cu") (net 31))
 (via (at 140.6 81.3) (size 0.6) (drill 0.3) (layers "F.Cu" "B.Cu") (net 31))
 (segment (start 140.6 81.3) (end 140.5 81.4) (width 0.2) (layer "B.Cu") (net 31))
 (segment (start 140.5 81.4) (end 140.5 86.8) (width 0.2) (layer "B.Cu") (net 31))
 (segment (start 131.34 82.66) (end 133.16 82.66) (width 0.2) (layer "F.Cu") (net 13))
 (segment (start 169.3 92.5) (end 132.3 92.5) (width 0.2) (layer "F.Cu") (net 13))
 (segment (start 185.2 92.6) (end 182 89.4) (width 0.2) (layer "F.Cu") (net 13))
 (segment (start 185.2 93.9) (end 185.2 92.6) (width 0.2) (layer "F.Cu") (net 13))
 (segment (start 227.6 93.5) (end 216.1 93.5) (width 0.2) (layer "F.Cu") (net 13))
 (segment (start 129.9 90.1) (end 129.9 84.1) (width 0.2) (layer "F.Cu") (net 13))
 (segment (start 213.1 99.7) (end 186.3 99.7) (width 0.2) (layer "F.Cu") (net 13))
 (segment (start 215 94.6) (end 215 97.8) (width 0.2) (layer "F.Cu") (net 13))
 (segment (start 182 89.4) (end 169.7 89.4) (width 0.2) (layer "F.Cu") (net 13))
 (segment (start 215 97.8) (end 213.1 99.7) (width 0.2) (layer "F.Cu") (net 13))
 (segment (start 216.1 93.5) (end 215 94.6) (width 0.2) (layer "F.Cu") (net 13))
 (segment (start 229.54 93.5) (end 232.8 90.24) (width 0.2) (layer "F.Cu") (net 13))
 (segment (start 129.9 84.1) (end 131.34 82.66) (width 0.2) (layer "F.Cu") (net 13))
 (segment (start 227.6 93.5) (end 229.54 93.5) (width 0.2) (layer "F.Cu") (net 13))
 (segment (start 132.3 92.5) (end 129.9 90.1) (width 0.2) (layer "F.Cu") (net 13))
 (segment (start 169.4 92.6) (end 169.3 92.5) (width 0.2) (layer "F.Cu") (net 13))
 (via (at 169.7 89.4) (size 0.6) (drill 0.3) (layers "F.Cu" "B.Cu") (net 13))
 (via (at 169.4 92.6) (size 0.6) (drill 0.3) (layers "F.Cu" "B.Cu") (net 13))
 (segment (start 169.7 89.4) (end 169.7 92.3) (width 0.2) (layer "B.Cu") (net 13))
 (segment (start 169.7 92.3) (end 169.4 92.6) (width 0.2) (layer "B.Cu") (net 13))
 (segment (start 170.71 84.2) (end 173.5 84.2) (width 0.2) (layer "F.Cu") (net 6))
 (segment (start 175.04 85.74) (end 175.04 86.28) (width 0.2) (layer "F.Cu") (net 6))
 (segment (start 173.5 84.2) (end 175.04 85.74) (width 0.2) (layer "F.Cu") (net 6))
 (segment (start 159.11 72.6) (end 170.71 84.2) (width 0.2) (layer "F.Cu") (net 6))
 (segment (start 156.57 73.17) (end 169.68 86.28) (width 0.2) (layer "F.Cu") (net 5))
 (segment (start 169.68 86.28) (end 172.5 86.28) (width 0.2) (layer "F.Cu") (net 5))
 (segment (start 156.57 72.6) (end 156.57 73.17) (width 0.2) (layer "F.Cu") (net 5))
 (segment (start 197 91.3) (end 208.9 91.3) (width 0.2) (layer "F.Cu") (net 1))
 (segment (start 208.9 91.3) (end 210.9 93.3) (width 0.2) (layer "F.Cu") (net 1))
 (segment (start 195.36 93.9) (end 195.36 92.94) (width 0.2) (layer "F.Cu") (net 1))
 (segment (start 195.36 94.56) (end 195.36 93.9) (width 0.2) (layer "F.Cu") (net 1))
 (segment (start 210.9 93.3) (end 210.9 94.7) (width 0.2) (layer "F.Cu") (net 1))
 (segment (start 197.9 97.1) (end 195.36 94.56) (width 0.2) (layer "F.Cu") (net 1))
 (segment (start 195.36 92.94) (end 197 91.3) (width 0.2) (layer "F.Cu") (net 1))
 (segment (start 174.5 90.4) (end 177.58 93.48) (width 0.2) (layer "F.Cu") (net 10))
 (segment (start 134.5 90.4) (end 174.5 90.4) (width 0.2) (layer "F.Cu") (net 10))
 (segment (start 133.16 89.06) (end 134.5 90.4) (width 0.2) (layer "F.Cu") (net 10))
 (segment (start 133.16 87.74) (end 133.16 89.06) (width 0.2) (layer "F.Cu") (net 10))
 (segment (start 177.58 93.48) (end 177.58 93.9) (width 0.2) (layer "F.Cu") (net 10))
 (segment (start 133.16 85.2) (end 131.6 85.2) (width 0.2) (layer "F.Cu") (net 9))
 (segment (start 131 85.8) (end 131 89.4) (width 0.2) (layer "F.Cu") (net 9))
 (segment (start 131.6 85.2) (end 131 85.8) (width 0.2) (layer "F.Cu") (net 9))
 (segment (start 175.04 93.24) (end 175.04 93.9) (width 0.2) (layer "F.Cu") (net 9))
 (segment (start 133.1 91.5) (end 173.3 91.5) (width 0.2) (layer "F.Cu") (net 9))
 (segment (start 173.3 91.5) (end 175.04 93.24) (width 0.2) (layer "F.Cu") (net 9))
 (segment (start 131 89.4) (end 133.1 91.5) (width 0.2) (layer "F.Cu") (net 9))
 (segment (start 192.82 93.08) (end 196.1 89.8) (width 0.2) (layer "F.Cu") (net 2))
 (segment (start 196.1 89.8) (end 210.9 89.8) (width 0.2) (layer "F.Cu") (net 2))
 (segment (start 192.75 97.1) (end 192.75 93.97) (width 0.2) (layer "F.Cu") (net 2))
 (segment (start 192.82 93.9) (end 192.82 93.08) (width 0.2) (layer "F.Cu") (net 2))
 (segment (start 192.75 93.97) (end 192.82 93.9) (width 0.2) (layer "F.Cu") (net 2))
 (segment (start 172.5 93.9) (end 172.5 96.28) (width 0.2) (layer "F.Cu") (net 8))
 (segment (start 214.1 97) (end 214.1 92.7) (width 0.2) (layer "F.Cu") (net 8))
 (segment (start 216.6 91.3) (end 223.1 91.3) (width 0.2) (layer "F.Cu") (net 8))
 (segment (start 173.62 97.4) (end 175.12 98.9) (width 0.2) (layer "F.Cu") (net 8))
 (segment (start 212.2 98.9) (end 214.1 97) (width 0.2) (layer "F.Cu") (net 8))
 (segment (start 172.5 96.28) (end 173.62 97.4) (width 0.2) (layer "F.Cu") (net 8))
 (segment (start 215.5 91.3) (end 216.6 91.3) (width 0.2) (layer "F.Cu") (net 8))
 (segment (start 175.12 98.9) (end 212.2 98.9) (width 0.2) (layer "F.Cu") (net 8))
 (segment (start 214.1 92.7) (end 215.5 91.3) (width 0.2) (layer "F.Cu") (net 8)))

